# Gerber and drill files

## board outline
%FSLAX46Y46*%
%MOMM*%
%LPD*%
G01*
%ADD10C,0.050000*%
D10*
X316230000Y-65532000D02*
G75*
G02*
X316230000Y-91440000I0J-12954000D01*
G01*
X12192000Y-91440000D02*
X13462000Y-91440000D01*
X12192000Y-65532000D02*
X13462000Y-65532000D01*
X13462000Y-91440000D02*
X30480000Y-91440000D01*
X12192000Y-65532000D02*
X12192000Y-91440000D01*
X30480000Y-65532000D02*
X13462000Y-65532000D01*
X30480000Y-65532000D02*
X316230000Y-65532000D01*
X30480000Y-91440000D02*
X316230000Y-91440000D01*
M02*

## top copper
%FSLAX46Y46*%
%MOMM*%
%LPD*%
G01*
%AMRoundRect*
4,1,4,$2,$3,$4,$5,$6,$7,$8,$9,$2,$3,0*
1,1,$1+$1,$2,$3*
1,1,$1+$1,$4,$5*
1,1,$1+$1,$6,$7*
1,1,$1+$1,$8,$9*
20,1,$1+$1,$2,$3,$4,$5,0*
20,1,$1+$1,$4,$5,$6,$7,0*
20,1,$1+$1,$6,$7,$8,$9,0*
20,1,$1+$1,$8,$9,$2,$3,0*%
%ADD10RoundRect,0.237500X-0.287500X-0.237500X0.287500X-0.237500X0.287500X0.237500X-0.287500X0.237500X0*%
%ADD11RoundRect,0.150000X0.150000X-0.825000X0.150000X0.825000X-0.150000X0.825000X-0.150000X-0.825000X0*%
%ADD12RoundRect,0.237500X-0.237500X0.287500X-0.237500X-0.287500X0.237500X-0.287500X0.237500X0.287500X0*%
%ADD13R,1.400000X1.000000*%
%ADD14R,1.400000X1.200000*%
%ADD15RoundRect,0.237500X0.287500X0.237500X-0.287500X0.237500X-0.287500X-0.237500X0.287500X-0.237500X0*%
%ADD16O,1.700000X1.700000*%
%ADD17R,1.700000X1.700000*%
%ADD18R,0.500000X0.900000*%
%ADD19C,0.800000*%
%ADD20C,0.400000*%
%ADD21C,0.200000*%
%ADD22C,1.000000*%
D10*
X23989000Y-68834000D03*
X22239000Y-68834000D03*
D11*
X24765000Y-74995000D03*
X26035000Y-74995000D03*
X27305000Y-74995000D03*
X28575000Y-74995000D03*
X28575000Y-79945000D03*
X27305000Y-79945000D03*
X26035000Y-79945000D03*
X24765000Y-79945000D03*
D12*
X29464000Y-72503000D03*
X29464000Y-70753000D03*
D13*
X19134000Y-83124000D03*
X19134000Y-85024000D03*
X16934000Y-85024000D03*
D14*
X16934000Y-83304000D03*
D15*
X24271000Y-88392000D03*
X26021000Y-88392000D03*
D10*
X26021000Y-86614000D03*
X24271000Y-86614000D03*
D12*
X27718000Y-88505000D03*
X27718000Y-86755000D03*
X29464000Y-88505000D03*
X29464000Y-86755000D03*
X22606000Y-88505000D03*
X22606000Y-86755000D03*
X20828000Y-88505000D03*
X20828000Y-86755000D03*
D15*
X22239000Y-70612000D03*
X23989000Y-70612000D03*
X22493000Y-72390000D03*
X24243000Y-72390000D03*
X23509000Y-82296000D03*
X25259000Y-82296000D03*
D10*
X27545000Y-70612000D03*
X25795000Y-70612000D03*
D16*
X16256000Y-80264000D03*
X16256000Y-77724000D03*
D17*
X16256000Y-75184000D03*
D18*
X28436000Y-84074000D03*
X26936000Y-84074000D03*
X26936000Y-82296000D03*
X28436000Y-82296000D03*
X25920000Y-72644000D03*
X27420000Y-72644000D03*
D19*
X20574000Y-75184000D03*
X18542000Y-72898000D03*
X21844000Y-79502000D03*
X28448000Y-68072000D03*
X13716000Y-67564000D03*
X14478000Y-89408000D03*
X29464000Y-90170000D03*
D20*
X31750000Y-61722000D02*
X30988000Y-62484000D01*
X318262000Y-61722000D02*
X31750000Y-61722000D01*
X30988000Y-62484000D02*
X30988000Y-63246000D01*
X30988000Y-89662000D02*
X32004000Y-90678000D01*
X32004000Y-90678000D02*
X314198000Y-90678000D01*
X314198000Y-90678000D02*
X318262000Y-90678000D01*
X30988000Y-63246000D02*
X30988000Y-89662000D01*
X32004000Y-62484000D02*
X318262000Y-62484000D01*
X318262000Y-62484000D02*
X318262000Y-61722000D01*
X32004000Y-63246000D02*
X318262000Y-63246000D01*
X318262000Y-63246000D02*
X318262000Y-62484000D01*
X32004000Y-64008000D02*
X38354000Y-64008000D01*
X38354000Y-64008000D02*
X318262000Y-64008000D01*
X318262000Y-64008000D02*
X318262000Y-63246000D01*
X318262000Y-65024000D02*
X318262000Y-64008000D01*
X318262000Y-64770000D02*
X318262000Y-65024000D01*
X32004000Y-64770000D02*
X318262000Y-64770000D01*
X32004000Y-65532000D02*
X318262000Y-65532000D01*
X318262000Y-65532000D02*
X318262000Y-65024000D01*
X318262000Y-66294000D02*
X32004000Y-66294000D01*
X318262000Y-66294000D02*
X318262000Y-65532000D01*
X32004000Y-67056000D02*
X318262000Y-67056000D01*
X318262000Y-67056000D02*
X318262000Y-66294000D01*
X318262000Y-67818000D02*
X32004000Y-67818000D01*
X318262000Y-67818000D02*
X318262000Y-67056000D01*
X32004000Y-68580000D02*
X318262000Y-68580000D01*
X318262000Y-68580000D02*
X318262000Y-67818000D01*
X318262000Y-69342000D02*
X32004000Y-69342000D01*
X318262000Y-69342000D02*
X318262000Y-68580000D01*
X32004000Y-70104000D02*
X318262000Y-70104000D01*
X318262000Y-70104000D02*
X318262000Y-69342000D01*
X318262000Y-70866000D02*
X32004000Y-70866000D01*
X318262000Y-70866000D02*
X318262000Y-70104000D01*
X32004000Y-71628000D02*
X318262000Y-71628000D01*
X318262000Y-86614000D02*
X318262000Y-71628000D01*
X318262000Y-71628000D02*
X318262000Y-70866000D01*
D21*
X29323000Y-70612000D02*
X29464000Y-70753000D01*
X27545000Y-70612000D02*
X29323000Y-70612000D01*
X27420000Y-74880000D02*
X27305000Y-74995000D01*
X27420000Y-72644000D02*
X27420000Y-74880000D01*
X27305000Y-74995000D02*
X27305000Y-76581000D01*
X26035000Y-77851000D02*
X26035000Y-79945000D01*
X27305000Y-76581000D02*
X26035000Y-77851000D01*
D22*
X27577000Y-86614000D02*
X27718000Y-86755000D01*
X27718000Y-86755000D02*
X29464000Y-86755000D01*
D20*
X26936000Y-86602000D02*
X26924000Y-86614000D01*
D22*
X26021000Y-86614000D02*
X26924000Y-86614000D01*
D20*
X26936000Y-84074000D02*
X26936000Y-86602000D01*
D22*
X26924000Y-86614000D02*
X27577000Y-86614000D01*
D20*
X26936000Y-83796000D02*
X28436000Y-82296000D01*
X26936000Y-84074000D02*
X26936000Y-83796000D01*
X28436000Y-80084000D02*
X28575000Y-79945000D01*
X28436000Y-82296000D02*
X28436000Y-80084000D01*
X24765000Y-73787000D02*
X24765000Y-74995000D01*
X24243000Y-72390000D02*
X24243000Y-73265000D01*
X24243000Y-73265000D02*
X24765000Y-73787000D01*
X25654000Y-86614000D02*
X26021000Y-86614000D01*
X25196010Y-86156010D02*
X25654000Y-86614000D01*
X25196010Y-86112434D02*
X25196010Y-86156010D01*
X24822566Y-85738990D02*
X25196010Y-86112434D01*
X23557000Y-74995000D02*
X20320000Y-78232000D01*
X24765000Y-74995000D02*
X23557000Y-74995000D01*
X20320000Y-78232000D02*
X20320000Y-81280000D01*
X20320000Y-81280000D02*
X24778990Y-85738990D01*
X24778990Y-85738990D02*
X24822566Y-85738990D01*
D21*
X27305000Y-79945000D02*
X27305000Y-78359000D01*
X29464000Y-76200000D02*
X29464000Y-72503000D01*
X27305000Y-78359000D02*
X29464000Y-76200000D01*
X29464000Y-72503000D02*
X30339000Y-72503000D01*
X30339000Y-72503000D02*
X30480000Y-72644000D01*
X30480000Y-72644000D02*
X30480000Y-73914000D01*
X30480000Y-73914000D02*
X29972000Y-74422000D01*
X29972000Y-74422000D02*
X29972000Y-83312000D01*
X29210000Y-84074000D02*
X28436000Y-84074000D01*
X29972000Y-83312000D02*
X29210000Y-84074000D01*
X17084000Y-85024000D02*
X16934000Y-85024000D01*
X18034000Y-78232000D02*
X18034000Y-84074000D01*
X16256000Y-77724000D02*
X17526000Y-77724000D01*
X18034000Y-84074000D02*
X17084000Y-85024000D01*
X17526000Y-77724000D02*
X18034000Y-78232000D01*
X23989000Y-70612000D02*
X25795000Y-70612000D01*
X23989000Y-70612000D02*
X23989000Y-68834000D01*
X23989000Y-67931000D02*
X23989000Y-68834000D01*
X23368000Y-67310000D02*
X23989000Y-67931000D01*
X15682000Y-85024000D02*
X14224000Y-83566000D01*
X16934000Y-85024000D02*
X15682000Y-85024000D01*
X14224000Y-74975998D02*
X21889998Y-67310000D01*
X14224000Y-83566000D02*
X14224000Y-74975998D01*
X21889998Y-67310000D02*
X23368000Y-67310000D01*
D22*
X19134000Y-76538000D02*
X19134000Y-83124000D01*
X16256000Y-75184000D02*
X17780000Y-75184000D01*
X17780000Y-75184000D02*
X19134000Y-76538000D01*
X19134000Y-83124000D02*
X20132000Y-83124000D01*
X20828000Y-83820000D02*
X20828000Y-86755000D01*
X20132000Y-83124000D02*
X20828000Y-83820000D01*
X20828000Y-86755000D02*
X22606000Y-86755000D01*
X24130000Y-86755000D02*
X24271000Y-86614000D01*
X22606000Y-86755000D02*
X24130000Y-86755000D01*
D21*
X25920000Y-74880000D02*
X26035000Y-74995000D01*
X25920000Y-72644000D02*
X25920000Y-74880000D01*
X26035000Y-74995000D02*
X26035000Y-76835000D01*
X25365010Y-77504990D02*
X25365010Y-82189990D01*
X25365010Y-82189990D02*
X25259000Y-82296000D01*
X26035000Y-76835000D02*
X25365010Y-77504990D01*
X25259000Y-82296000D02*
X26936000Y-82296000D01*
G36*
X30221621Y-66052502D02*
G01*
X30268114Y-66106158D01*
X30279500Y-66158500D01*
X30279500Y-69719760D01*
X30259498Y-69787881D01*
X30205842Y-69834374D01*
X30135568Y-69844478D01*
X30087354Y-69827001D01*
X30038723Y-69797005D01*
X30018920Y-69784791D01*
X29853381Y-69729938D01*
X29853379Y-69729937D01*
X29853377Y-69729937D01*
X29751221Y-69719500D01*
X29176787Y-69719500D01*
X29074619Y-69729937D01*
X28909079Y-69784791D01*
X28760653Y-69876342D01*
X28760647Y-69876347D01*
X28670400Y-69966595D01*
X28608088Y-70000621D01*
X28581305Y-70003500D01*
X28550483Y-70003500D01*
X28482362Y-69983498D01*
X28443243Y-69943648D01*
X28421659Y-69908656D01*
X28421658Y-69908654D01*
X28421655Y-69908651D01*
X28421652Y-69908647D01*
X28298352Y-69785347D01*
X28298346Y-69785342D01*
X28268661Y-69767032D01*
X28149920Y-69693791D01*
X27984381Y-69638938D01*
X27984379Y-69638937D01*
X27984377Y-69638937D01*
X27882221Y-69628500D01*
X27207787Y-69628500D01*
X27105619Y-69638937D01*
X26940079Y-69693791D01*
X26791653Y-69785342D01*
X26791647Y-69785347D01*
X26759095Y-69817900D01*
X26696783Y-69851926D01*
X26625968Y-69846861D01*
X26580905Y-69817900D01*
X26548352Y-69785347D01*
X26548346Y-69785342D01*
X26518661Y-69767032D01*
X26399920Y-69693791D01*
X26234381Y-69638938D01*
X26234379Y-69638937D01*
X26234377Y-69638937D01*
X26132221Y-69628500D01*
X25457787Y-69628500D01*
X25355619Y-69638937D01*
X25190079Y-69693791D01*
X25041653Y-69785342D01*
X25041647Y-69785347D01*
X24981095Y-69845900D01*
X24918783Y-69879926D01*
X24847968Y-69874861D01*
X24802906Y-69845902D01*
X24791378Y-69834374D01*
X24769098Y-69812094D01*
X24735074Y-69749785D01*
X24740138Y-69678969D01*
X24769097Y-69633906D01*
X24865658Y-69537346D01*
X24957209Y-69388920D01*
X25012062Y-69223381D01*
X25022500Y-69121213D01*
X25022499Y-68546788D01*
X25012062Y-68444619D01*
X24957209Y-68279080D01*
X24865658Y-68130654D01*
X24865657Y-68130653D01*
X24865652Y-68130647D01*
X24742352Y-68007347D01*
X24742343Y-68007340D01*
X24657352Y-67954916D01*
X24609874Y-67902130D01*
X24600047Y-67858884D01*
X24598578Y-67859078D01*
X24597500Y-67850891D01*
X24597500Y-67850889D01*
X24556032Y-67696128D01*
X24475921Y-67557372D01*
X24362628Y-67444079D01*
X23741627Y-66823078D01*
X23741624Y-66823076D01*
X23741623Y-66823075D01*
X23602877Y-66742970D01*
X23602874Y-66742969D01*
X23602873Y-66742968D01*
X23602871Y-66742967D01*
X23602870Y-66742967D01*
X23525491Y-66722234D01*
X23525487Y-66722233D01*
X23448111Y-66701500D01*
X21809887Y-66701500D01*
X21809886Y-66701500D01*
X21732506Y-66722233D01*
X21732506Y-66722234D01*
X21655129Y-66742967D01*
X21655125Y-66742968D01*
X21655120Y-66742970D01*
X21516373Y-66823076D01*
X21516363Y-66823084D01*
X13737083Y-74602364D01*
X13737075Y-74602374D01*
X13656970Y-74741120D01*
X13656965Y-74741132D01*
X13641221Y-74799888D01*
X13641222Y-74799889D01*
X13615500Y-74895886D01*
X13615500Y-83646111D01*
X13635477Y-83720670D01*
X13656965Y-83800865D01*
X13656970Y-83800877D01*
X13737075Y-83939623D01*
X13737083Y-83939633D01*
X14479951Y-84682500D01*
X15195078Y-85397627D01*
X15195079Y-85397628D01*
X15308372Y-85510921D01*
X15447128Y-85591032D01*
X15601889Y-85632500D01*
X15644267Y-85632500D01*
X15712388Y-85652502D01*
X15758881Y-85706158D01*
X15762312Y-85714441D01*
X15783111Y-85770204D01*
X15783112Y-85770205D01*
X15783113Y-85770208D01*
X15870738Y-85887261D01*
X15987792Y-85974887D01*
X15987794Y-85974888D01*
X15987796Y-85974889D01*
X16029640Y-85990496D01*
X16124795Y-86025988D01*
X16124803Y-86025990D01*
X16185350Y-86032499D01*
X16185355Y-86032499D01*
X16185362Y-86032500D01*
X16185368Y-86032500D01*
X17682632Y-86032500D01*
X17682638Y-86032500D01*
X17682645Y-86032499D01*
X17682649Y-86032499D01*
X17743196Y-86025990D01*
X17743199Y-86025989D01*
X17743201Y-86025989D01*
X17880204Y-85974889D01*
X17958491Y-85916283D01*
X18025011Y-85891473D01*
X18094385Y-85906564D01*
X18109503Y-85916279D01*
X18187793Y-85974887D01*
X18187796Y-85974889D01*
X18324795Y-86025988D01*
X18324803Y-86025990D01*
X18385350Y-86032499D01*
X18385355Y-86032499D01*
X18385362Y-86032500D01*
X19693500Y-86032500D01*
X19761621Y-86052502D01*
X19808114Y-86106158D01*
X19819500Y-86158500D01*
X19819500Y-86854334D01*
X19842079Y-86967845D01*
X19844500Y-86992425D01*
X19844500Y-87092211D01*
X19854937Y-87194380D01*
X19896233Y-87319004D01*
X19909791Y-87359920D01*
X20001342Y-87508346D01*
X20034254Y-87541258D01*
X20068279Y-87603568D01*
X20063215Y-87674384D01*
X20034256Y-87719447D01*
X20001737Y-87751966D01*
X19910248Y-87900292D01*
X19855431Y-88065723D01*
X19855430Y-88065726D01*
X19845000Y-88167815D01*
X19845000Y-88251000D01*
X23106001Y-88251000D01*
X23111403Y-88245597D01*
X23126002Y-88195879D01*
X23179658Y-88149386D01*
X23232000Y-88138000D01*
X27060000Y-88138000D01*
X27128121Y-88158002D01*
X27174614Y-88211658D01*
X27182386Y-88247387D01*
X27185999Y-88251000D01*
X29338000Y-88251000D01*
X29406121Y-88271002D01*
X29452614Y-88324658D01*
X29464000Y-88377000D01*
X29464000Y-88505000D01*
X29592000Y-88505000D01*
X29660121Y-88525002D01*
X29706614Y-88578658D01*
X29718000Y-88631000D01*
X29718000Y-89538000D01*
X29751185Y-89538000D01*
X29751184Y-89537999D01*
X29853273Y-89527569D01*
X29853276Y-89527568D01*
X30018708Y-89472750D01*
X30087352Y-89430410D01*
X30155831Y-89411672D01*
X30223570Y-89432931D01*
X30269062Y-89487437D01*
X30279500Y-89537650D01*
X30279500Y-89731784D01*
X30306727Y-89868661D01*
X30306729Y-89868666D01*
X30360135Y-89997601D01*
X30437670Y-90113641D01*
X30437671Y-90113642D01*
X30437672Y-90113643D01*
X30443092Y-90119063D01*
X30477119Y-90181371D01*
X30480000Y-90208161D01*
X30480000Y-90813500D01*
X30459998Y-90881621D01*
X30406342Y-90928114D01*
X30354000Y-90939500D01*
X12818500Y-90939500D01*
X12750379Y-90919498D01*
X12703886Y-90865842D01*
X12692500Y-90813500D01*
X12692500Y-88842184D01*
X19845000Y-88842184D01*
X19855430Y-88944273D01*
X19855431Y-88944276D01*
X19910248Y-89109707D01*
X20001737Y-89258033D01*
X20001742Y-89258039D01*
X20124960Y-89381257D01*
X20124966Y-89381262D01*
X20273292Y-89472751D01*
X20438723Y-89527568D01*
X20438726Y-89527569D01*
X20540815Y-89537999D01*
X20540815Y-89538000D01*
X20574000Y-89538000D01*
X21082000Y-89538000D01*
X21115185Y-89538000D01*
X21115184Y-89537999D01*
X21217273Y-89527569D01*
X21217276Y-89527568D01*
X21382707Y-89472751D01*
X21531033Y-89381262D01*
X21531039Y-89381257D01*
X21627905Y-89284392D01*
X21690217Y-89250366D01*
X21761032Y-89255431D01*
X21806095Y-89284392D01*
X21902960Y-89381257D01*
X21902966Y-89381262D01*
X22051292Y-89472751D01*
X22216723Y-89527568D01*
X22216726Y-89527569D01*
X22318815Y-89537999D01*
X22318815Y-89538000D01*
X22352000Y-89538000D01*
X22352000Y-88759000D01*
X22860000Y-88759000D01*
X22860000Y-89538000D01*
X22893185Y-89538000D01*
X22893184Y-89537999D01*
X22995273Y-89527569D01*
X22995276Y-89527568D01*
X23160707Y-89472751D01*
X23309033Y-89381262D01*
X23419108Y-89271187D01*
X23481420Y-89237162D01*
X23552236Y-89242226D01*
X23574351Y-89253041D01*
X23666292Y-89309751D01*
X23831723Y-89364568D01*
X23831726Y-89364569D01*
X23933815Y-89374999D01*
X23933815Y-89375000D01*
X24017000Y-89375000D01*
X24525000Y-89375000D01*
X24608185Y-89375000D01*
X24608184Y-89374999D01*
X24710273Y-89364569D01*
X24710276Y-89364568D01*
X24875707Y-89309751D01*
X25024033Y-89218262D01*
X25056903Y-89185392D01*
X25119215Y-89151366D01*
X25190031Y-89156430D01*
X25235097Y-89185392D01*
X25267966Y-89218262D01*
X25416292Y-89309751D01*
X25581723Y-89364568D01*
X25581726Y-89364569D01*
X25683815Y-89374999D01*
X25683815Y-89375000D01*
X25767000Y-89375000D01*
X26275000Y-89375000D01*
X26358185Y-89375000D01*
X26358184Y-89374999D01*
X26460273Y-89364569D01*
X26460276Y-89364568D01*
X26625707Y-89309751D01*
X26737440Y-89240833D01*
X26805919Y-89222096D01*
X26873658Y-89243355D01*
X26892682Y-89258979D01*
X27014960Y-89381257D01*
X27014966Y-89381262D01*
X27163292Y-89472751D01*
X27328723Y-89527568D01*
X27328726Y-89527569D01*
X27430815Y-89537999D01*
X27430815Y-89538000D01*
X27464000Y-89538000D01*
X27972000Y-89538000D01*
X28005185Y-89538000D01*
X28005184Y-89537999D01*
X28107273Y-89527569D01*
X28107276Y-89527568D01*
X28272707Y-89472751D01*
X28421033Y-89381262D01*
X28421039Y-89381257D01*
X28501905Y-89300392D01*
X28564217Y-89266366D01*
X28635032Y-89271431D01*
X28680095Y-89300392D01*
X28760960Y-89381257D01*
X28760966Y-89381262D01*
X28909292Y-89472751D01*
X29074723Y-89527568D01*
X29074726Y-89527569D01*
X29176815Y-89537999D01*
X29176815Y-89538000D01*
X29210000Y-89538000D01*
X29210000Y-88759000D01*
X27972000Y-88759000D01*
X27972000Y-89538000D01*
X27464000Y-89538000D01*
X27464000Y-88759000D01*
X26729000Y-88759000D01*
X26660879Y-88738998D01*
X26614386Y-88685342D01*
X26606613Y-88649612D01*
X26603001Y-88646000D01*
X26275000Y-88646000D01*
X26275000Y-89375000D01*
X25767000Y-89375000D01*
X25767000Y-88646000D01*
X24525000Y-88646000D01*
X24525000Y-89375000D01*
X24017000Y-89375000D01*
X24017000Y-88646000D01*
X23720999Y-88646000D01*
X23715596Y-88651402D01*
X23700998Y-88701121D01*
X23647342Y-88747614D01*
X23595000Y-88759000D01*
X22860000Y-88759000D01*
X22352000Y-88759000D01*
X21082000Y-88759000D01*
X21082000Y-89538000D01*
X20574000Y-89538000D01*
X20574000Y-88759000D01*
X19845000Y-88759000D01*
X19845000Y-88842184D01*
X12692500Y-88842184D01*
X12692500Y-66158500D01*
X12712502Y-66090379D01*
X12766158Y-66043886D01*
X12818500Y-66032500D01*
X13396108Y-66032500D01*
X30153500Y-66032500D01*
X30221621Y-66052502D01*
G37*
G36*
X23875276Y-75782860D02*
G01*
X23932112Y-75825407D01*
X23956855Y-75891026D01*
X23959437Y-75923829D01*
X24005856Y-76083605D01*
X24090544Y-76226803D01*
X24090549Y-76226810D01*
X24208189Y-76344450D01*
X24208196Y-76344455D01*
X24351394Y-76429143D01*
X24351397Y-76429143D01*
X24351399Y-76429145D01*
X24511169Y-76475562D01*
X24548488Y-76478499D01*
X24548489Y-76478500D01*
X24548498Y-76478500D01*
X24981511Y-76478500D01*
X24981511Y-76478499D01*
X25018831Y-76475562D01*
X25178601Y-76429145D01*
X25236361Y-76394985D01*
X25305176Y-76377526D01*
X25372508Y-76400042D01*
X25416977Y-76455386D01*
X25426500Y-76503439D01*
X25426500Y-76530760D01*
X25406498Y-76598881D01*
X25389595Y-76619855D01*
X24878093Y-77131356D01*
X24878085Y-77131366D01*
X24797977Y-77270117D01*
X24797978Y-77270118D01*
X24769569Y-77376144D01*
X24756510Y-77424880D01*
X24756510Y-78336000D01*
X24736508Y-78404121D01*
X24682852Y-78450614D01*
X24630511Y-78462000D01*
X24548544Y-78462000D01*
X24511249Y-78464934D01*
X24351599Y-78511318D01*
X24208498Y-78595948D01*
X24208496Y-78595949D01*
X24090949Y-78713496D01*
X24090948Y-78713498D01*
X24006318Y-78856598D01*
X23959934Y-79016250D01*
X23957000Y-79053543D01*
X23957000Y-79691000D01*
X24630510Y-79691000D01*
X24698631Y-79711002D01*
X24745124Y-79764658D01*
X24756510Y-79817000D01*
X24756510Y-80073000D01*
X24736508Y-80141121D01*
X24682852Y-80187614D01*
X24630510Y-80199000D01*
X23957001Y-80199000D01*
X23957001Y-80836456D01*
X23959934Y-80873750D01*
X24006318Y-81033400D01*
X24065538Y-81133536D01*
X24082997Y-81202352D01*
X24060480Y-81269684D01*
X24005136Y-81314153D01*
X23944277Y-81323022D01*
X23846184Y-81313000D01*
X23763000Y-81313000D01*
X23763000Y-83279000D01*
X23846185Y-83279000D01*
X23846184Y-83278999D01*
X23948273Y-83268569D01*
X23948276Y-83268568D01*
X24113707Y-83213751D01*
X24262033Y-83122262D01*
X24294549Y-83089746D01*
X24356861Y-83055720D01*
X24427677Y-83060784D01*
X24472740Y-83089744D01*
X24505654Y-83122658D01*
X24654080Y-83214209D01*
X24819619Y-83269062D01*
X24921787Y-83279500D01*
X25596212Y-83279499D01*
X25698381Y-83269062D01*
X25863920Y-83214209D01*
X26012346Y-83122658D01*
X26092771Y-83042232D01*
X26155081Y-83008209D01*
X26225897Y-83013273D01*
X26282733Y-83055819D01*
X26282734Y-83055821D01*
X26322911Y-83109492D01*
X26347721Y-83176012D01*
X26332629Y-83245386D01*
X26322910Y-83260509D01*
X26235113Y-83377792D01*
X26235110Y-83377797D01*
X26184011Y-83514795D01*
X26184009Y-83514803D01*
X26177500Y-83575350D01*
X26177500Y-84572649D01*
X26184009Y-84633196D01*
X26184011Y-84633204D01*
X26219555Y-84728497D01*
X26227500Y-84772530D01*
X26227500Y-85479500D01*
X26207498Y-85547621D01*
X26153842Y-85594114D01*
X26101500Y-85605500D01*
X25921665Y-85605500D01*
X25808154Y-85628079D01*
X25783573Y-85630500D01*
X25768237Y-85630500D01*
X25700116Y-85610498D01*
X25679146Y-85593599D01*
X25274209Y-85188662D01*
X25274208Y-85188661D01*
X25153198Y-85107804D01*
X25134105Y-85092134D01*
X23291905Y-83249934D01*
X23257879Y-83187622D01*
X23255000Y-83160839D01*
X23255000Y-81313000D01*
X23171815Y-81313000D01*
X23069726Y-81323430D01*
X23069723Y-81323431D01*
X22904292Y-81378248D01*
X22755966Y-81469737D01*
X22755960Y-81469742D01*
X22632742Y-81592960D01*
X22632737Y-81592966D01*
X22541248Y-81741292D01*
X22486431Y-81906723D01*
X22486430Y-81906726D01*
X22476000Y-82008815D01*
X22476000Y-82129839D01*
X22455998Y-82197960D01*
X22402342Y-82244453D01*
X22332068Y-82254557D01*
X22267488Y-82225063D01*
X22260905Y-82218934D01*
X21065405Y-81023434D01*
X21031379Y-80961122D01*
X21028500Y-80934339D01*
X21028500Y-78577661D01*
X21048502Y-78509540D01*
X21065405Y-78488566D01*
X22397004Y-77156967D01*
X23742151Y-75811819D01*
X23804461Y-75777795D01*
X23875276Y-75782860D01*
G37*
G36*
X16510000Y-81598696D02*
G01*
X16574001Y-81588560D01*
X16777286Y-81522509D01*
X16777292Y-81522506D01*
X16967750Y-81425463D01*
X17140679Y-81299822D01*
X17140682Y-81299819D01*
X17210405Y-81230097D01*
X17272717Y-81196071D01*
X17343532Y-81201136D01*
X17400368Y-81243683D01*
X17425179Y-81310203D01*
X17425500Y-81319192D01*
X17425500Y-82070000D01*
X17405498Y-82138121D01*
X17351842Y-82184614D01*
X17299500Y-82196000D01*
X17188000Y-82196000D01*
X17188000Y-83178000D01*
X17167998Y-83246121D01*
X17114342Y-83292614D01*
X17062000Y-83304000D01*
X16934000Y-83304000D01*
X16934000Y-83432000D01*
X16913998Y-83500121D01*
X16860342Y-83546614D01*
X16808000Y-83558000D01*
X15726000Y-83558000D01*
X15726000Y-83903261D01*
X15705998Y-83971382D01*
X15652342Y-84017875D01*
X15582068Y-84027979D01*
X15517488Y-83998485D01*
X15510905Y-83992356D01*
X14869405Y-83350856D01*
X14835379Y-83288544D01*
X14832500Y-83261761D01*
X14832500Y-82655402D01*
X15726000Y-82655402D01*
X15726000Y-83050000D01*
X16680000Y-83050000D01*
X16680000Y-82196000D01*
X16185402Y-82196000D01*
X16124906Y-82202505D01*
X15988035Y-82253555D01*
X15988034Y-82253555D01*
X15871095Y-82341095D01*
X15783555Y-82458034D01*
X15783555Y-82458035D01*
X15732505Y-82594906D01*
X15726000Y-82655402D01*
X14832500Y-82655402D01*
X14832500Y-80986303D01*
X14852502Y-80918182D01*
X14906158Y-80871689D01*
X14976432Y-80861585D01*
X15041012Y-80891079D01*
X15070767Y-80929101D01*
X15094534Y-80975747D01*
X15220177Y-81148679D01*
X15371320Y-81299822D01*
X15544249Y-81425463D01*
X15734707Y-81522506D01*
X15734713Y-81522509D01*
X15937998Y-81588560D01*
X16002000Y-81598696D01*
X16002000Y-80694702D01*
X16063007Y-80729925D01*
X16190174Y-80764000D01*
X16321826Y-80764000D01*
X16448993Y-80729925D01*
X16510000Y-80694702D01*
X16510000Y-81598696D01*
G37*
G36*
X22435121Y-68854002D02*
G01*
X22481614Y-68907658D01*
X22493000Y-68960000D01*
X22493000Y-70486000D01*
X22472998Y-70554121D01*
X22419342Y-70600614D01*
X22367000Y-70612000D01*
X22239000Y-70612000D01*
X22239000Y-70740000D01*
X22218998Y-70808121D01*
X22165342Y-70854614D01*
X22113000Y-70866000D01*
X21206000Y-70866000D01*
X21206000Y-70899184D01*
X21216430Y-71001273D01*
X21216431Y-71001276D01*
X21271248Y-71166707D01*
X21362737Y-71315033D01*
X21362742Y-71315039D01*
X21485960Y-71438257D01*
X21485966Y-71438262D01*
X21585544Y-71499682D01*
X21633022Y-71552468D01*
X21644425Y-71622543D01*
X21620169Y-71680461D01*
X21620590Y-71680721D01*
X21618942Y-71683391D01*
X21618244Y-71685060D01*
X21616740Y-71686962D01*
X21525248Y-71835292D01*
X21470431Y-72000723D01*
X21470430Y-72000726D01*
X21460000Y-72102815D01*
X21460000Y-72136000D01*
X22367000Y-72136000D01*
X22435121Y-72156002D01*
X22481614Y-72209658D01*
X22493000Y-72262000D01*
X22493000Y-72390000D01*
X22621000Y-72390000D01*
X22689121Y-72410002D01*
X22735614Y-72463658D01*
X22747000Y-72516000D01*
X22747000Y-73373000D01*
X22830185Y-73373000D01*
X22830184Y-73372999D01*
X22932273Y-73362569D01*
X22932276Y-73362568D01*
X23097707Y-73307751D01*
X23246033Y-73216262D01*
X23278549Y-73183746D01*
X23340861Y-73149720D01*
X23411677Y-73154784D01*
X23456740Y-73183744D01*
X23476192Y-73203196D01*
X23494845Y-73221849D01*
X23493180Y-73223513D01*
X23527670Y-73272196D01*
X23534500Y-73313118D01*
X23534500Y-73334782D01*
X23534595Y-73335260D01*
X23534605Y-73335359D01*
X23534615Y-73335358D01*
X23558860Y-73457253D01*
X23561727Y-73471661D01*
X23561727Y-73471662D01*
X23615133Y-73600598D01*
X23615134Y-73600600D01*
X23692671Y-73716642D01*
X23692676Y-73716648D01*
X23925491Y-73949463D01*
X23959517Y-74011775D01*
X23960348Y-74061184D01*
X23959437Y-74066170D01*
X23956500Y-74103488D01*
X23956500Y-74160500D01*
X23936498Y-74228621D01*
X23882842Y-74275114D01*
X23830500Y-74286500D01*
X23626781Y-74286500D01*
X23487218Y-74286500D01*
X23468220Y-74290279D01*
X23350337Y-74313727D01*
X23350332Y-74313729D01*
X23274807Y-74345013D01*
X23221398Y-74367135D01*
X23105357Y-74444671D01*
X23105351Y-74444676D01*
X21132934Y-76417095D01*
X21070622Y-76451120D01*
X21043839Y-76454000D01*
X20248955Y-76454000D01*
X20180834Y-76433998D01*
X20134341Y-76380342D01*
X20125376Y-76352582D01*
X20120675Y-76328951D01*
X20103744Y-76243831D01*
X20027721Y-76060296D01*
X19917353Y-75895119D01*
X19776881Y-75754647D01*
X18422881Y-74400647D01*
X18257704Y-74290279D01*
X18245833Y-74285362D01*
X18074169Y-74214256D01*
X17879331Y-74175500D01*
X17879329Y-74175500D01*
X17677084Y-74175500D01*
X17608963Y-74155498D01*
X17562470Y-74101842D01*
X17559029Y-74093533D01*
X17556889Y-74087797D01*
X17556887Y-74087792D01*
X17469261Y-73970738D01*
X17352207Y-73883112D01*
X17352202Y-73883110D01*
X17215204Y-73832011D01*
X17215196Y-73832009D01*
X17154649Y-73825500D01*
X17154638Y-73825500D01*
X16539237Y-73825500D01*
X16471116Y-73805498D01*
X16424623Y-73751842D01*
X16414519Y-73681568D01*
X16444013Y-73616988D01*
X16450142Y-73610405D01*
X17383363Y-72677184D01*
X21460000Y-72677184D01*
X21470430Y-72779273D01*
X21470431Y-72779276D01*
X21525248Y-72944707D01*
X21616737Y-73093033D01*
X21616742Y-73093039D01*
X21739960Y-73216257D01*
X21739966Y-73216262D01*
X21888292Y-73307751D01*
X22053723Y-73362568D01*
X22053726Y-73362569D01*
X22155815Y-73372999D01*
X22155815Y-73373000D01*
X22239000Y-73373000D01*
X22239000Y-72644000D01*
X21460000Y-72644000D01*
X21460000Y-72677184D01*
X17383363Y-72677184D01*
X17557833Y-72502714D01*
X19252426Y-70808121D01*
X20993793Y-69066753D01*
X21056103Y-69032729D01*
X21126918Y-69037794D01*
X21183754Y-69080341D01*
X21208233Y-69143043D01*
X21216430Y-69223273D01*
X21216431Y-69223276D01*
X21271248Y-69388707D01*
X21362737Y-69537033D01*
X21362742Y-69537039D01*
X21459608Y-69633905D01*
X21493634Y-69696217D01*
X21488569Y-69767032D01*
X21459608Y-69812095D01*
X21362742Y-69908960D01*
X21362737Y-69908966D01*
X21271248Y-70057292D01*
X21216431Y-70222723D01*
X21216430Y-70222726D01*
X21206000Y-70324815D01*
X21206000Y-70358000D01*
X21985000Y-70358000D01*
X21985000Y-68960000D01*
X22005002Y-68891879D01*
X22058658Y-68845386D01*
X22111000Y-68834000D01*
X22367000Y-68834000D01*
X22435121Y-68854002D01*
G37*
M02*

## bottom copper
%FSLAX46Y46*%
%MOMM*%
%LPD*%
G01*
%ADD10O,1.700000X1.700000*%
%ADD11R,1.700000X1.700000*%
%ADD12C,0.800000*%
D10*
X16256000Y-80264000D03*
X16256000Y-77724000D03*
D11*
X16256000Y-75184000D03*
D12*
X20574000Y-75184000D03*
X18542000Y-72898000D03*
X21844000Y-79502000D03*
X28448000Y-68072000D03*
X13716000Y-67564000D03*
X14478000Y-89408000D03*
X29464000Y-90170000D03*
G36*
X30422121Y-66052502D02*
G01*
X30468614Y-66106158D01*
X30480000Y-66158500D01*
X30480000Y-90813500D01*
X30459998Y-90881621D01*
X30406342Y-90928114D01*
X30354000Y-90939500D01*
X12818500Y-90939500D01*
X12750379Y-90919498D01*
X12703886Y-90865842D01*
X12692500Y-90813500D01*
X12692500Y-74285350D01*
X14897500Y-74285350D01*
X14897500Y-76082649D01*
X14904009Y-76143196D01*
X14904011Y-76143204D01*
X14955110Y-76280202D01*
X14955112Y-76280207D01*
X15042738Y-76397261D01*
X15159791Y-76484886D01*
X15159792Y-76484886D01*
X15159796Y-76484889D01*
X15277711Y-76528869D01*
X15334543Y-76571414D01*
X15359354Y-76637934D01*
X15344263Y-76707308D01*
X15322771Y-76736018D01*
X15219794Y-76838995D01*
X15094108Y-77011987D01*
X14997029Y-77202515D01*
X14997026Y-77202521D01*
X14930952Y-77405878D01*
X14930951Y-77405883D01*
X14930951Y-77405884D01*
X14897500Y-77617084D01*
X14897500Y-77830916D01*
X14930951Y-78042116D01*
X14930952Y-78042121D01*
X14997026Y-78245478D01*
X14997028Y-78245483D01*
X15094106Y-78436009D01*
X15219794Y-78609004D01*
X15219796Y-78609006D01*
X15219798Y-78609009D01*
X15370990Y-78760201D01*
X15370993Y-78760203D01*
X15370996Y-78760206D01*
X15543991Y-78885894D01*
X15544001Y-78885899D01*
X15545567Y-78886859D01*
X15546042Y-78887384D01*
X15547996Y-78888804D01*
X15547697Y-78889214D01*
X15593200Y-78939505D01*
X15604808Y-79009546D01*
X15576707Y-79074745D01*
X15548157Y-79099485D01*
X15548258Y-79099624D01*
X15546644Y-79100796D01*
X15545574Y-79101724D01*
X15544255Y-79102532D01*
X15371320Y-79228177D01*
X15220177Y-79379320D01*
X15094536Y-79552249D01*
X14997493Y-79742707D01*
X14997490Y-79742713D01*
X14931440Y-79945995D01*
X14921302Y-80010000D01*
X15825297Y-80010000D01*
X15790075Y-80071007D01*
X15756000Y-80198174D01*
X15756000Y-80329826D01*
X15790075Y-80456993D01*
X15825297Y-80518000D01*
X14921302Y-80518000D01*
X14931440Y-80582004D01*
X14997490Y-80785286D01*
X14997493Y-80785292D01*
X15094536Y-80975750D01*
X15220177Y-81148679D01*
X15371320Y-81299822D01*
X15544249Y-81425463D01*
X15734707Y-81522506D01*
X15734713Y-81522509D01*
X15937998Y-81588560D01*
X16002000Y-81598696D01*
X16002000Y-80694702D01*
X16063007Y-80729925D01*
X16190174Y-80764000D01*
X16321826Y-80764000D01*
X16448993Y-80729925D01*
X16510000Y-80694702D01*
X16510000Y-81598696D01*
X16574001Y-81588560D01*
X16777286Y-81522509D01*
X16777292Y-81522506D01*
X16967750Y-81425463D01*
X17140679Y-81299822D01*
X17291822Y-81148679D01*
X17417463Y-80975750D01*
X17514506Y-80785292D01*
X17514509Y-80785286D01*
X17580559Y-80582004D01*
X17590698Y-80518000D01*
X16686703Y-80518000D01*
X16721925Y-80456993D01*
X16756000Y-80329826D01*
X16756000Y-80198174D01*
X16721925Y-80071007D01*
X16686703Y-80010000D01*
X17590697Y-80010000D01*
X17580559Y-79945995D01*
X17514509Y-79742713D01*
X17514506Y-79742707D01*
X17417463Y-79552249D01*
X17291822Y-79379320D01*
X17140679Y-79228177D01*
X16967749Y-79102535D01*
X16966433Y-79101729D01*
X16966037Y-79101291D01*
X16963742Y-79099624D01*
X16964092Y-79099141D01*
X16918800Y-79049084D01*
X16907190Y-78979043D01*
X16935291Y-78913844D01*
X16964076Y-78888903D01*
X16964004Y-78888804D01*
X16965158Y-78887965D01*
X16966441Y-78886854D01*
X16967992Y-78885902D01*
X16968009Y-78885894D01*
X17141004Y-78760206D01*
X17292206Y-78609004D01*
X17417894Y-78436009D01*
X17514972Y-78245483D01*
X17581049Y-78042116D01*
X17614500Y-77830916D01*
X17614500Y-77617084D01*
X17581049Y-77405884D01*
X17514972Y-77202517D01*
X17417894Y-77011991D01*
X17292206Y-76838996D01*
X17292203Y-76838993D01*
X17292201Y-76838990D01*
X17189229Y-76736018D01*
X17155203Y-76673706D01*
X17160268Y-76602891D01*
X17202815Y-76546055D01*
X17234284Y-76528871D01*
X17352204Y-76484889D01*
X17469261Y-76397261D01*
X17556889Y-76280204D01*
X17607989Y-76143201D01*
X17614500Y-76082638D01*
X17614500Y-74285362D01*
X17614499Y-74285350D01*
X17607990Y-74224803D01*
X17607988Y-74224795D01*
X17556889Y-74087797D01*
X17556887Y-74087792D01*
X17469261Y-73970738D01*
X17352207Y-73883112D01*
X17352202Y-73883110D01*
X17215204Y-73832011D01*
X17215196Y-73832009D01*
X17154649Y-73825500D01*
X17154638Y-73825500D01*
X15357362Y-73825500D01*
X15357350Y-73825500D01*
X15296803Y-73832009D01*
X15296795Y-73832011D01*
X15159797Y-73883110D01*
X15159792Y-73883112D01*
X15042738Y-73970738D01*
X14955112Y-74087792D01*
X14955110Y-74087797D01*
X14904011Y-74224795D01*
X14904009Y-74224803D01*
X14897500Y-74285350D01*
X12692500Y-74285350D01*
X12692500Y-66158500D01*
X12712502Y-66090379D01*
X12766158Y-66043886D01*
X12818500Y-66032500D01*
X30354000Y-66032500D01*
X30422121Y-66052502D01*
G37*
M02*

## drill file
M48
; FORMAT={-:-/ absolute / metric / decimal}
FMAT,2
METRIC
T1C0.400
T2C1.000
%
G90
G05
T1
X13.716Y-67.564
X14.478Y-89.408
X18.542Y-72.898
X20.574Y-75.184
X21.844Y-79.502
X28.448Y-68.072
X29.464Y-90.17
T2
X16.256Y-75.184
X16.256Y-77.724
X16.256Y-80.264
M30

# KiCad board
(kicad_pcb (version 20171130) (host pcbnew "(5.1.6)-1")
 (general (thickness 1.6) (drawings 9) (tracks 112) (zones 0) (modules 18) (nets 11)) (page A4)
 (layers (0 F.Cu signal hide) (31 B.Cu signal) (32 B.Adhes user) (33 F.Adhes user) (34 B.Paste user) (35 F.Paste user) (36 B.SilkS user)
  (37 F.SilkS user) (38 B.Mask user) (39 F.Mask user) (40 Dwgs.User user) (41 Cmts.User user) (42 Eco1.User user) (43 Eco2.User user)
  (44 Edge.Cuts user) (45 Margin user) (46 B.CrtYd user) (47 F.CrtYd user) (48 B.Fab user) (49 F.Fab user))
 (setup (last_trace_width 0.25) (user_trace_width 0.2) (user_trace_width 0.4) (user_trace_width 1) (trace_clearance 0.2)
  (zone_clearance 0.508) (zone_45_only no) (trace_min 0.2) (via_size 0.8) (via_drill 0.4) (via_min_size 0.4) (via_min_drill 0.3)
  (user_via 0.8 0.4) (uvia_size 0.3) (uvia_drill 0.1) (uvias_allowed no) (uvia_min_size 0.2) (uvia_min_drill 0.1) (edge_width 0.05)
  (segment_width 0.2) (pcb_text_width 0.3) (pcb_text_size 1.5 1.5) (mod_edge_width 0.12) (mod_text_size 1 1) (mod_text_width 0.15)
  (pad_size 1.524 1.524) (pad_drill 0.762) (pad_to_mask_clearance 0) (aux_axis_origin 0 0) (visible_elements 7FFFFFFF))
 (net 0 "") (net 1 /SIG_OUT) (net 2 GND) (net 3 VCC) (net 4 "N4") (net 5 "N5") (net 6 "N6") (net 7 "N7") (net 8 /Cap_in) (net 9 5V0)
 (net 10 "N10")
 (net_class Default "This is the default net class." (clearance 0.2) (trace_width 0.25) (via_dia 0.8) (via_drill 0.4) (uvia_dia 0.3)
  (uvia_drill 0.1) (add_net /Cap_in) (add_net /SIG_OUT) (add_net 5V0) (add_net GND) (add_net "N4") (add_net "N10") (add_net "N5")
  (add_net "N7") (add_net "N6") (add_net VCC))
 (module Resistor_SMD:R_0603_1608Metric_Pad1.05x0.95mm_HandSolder (layer F.Cu) (at 23.114 68.834)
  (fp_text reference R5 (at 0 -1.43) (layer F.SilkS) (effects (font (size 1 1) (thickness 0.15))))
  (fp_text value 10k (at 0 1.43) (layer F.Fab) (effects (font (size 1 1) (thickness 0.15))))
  (pad 2 smd roundrect (at 0.875 0) (size 1.05 0.95) (layers F.Cu F.Paste F.Mask) (roundrect_rratio 0.25) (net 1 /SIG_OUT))
  (pad 1 smd roundrect (at -0.875 0) (size 1.05 0.95) (layers F.Cu F.Paste F.Mask) (roundrect_rratio 0.25) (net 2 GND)))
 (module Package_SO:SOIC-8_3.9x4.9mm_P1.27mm (layer F.Cu) (at 26.67 77.47 90)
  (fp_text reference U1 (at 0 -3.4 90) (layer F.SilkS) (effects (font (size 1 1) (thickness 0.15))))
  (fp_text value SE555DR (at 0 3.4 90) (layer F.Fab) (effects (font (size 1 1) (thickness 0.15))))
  (pad 8 smd roundrect (at 2.475 -1.905 90) (size 1.95 0.6) (layers F.Cu F.Paste F.Mask) (roundrect_rratio 0.25) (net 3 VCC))
  (pad 7 smd roundrect (at 2.475 -0.635 90) (size 1.95 0.6) (layers F.Cu F.Paste F.Mask) (roundrect_rratio 0.25) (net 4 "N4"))
  (pad 6 smd roundrect (at 2.475 0.635 90) (size 1.95 0.6) (layers F.Cu F.Paste F.Mask) (roundrect_rratio 0.25) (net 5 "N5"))
  (pad 5 smd roundrect (at 2.475 1.905 90) (size 1.95 0.6) (layers F.Cu F.Paste F.Mask) (roundrect_rratio 0.25) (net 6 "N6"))
  (pad 4 smd roundrect (at -2.475 1.905 90) (size 1.95 0.6) (layers F.Cu F.Paste F.Mask) (roundrect_rratio 0.25) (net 3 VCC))
  (pad 3 smd roundrect (at -2.475 0.635 90) (size 1.95 0.6) (layers F.Cu F.Paste F.Mask) (roundrect_rratio 0.25) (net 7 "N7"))
  (pad 2 smd roundrect (at -2.475 -0.635 90) (size 1.95 0.6) (layers F.Cu F.Paste F.Mask) (roundrect_rratio 0.25) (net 5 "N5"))
  (pad 1 smd roundrect (at -2.475 -1.905 90) (size 1.95 0.6) (layers F.Cu F.Paste F.Mask) (roundrect_rratio 0.25) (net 2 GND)))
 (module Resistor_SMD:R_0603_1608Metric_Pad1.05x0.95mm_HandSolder (layer F.Cu) (at 29.464 71.628 270)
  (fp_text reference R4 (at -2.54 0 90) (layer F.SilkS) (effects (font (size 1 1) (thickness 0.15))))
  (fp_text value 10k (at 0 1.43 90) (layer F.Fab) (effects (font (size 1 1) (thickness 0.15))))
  (pad 2 smd roundrect (at 0.875 0 270) (size 1.05 0.95) (layers F.Cu F.Paste F.Mask) (roundrect_rratio 0.25) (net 7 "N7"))
  (pad 1 smd roundrect (at -0.875 0 270) (size 1.05 0.95) (layers F.Cu F.Paste F.Mask) (roundrect_rratio 0.25) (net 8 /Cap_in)))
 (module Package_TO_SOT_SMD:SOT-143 (layer F.Cu) (at 18.034 84.074)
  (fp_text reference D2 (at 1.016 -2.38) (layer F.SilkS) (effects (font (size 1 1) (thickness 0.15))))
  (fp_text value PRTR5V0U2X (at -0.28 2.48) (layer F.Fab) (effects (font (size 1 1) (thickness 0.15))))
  (pad 4 smd rect (at 1.1 -0.95 270) (size 1 1.4) (layers F.Cu F.Paste F.Mask) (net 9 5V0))
  (pad 3 smd rect (at 1.1 0.95 270) (size 1 1.4) (layers F.Cu F.Paste F.Mask) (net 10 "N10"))
  (pad 2 smd rect (at -1.1 0.95 270) (size 1 1.4) (layers F.Cu F.Paste F.Mask) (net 1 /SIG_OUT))
  (pad 1 smd rect (at -1.1 -0.77 270) (size 1.2 1.4) (layers F.Cu F.Paste F.Mask) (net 2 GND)))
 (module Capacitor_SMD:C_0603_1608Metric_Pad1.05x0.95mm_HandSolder (layer F.Cu) (at 25.146 88.392 180)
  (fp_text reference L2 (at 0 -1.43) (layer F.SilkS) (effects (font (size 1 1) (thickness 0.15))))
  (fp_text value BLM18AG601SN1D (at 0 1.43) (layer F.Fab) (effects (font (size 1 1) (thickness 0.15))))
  (pad 2 smd roundrect (at 0.875 0 180) (size 1.05 0.95) (layers F.Cu F.Paste F.Mask) (roundrect_rratio 0.25) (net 2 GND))
  (pad 1 smd roundrect (at -0.875 0 180) (size 1.05 0.95) (layers F.Cu F.Paste F.Mask) (roundrect_rratio 0.25) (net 2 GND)))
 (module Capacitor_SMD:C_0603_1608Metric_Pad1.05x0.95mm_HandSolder (layer F.Cu) (at 25.146 86.614)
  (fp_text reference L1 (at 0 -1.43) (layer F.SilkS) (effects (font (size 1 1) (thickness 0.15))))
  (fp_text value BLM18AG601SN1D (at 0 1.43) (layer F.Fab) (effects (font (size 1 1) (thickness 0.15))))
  (pad 2 smd roundrect (at 0.875 0) (size 1.05 0.95) (layers F.Cu F.Paste F.Mask) (roundrect_rratio 0.25) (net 3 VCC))
  (pad 1 smd roundrect (at -0.875 0) (size 1.05 0.95) (layers F.Cu F.Paste F.Mask) (roundrect_rratio 0.25) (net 9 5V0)))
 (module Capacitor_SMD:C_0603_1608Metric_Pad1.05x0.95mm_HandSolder (layer F.Cu) (at 27.718 87.63 270)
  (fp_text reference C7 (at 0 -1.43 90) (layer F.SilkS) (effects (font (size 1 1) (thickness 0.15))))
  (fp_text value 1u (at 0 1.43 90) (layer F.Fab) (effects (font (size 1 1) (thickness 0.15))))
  (pad 2 smd roundrect (at 0.875 0 270) (size 1.05 0.95) (layers F.Cu F.Paste F.Mask) (roundrect_rratio 0.25) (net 2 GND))
  (pad 1 smd roundrect (at -0.875 0 270) (size 1.05 0.95) (layers F.Cu F.Paste F.Mask) (roundrect_rratio 0.25) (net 3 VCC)))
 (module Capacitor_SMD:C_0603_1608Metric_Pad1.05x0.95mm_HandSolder (layer F.Cu) (at 29.464 87.63 270)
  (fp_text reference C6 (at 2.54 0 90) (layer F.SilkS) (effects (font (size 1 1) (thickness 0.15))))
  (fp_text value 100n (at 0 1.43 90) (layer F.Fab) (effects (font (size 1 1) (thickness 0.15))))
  (pad 2 smd roundrect (at 0.875 0 270) (size 1.05 0.95) (layers F.Cu F.Paste F.Mask) (roundrect_rratio 0.25) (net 2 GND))
  (pad 1 smd roundrect (at -0.875 0 270) (size 1.05 0.95) (layers F.Cu F.Paste F.Mask) (roundrect_rratio 0.25) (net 3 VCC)))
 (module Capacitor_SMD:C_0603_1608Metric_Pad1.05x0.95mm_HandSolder (layer F.Cu) (at 22.606 87.63 270)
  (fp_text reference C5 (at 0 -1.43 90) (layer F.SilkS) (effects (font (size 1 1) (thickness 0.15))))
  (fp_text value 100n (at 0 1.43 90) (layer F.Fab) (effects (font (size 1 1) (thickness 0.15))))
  (pad 2 smd roundrect (at 0.875 0 270) (size 1.05 0.95) (layers F.Cu F.Paste F.Mask) (roundrect_rratio 0.25) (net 2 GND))
  (pad 1 smd roundrect (at -0.875 0 270) (size 1.05 0.95) (layers F.Cu F.Paste F.Mask) (roundrect_rratio 0.25) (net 9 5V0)))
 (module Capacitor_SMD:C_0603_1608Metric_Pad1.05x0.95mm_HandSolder (layer F.Cu) (at 20.828 87.63 270)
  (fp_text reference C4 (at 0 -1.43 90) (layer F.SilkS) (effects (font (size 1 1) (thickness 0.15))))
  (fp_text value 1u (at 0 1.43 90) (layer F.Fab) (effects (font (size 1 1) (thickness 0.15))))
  (pad 2 smd roundrect (at 0.875 0 270) (size 1.05 0.95) (layers F.Cu F.Paste F.Mask) (roundrect_rratio 0.25) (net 2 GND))
  (pad 1 smd roundrect (at -0.875 0 270) (size 1.05 0.95) (layers F.Cu F.Paste F.Mask) (roundrect_rratio 0.25) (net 9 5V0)))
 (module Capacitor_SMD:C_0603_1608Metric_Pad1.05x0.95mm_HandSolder (layer F.Cu) (at 23.114 70.612 180)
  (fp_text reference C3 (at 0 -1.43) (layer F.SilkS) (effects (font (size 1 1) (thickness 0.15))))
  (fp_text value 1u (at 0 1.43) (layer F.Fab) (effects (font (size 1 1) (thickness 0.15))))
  (pad 2 smd roundrect (at 0.875 0 180) (size 1.05 0.95) (layers F.Cu F.Paste F.Mask) (roundrect_rratio 0.25) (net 2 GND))
  (pad 1 smd roundrect (at -0.875 0 180) (size 1.05 0.95) (layers F.Cu F.Paste F.Mask) (roundrect_rratio 0.25) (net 1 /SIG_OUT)))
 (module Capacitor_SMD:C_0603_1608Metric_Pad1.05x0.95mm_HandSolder (layer F.Cu) (at 23.368 72.39 180)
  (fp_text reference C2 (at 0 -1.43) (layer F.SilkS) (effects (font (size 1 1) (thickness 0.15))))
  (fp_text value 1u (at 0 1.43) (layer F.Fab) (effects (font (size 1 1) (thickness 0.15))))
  (pad 2 smd roundrect (at 0.875 0 180) (size 1.05 0.95) (layers F.Cu F.Paste F.Mask) (roundrect_rratio 0.25) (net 2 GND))
  (pad 1 smd roundrect (at -0.875 0 180) (size 1.05 0.95) (layers F.Cu F.Paste F.Mask) (roundrect_rratio 0.25) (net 3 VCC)))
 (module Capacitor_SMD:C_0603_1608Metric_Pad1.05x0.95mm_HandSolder (layer F.Cu) (at 24.384 82.296 180)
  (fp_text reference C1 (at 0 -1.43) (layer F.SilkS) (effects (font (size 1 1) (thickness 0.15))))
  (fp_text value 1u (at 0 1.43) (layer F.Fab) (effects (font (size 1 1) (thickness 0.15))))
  (pad 2 smd roundrect (at 0.875 0 180) (size 1.05 0.95) (layers F.Cu F.Paste F.Mask) (roundrect_rratio 0.25) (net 2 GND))
  (pad 1 smd roundrect (at -0.875 0 180) (size 1.05 0.95) (layers F.Cu F.Paste F.Mask) (roundrect_rratio 0.25) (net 4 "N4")))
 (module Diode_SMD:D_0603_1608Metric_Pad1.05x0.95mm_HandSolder (layer F.Cu) (at 26.67 70.612)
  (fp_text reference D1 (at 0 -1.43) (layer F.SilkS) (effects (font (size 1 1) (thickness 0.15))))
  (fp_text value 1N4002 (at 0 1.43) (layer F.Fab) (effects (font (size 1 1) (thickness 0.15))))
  (pad 2 smd roundrect (at 0.875 0) (size 1.05 0.95) (layers F.Cu F.Paste F.Mask) (roundrect_rratio 0.25) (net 8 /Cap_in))
  (pad 1 smd roundrect (at -0.875 0) (size 1.05 0.95) (layers F.Cu F.Paste F.Mask) (roundrect_rratio 0.25) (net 1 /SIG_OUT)))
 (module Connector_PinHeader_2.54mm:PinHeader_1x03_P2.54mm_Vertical (layer F.Cu) (at 16.256 75.184)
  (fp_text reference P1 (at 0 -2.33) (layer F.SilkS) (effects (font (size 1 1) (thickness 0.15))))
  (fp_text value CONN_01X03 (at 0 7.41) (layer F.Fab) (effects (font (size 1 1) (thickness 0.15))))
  (pad 3 thru_hole oval (at 0 5.08) (size 1.7 1.7) (drill 1) (layers *.Cu *.Mask) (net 2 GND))
  (pad 2 thru_hole oval (at 0 2.54) (size 1.7 1.7) (drill 1) (layers *.Cu *.Mask) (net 1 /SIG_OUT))
  (pad 1 thru_hole rect (at 0 0) (size 1.7 1.7) (drill 1) (layers *.Cu *.Mask) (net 9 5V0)))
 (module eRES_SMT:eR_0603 (layer F.Cu) (at 27.686 84.074)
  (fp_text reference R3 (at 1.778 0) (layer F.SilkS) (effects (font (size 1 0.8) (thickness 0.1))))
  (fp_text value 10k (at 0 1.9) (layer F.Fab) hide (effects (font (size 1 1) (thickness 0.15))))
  (pad 2 smd rect (at 0.75 0) (size 0.5 0.9) (layers F.Cu F.Paste F.Mask) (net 7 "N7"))
  (pad 1 smd rect (at -0.75 0) (size 0.5 0.9) (layers F.Cu F.Paste F.Mask) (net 3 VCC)))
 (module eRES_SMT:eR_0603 (layer F.Cu) (at 27.686 82.296 180)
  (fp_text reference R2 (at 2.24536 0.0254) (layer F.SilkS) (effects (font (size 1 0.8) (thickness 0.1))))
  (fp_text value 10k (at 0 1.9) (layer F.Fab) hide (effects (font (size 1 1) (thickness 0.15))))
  (pad 2 smd rect (at 0.75 0 180) (size 0.5 0.9) (layers F.Cu F.Paste F.Mask) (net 4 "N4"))
  (pad 1 smd rect (at -0.75 0 180) (size 0.5 0.9) (layers F.Cu F.Paste F.Mask) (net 3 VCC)))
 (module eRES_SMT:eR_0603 (layer F.Cu) (at 26.67 72.644 180)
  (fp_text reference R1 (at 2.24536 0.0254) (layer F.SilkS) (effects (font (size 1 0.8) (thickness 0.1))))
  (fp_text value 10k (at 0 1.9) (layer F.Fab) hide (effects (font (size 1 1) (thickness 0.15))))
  (pad 2 smd rect (at 0.75 0 180) (size 0.5 0.9) (layers F.Cu F.Paste F.Mask) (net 4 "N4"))
  (pad 1 smd rect (at -0.75 0 180) (size 0.5 0.9) (layers F.Cu F.Paste F.Mask) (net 5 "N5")))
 (gr_arc (start 316.23 78.486) (end 316.23 91.44) (angle -180) (layer Edge.Cuts) (width 0.05))
 (gr_line (start 12.192 91.44) (end 13.462 91.44) (layer Edge.Cuts) (width 0.05))
 (gr_line (start 12.192 65.532) (end 13.462 65.532) (layer Edge.Cuts) (width 0.05))
 (gr_line (start 13.462 91.44) (end 30.48 91.44) (layer Edge.Cuts) (width 0.05))
 (gr_line (start 12.192 65.532) (end 12.192 91.44) (layer Edge.Cuts) (width 0.05))
 (gr_line (start 30.48 65.532) (end 13.462 65.532) (layer Edge.Cuts) (width 0.05))
 (gr_line (start 30.48 65.532) (end 316.23 65.532) (layer Edge.Cuts) (width 0.05))
 (gr_line (start 30.48 91.44) (end 316.23 91.44) (layer Edge.Cuts) (width 0.05))
 (segment (start 31.75 61.722) (end 30.988 62.484) (width 0.4) (layer F.Cu) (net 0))
 (segment (start 318.262 61.722) (end 31.75 61.722) (width 0.4) (layer F.Cu) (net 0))
 (segment (start 30.988 62.484) (end 30.988 63.246) (width 0.4) (layer F.Cu) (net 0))
 (segment (start 30.988 89.662) (end 32.004 90.678) (width 0.4) (layer F.Cu) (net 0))
 (segment (start 32.004 90.678) (end 314.198 90.678) (width 0.4) (layer F.Cu) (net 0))
 (segment (start 314.198 90.678) (end 318.262 90.678) (width 0.4) (layer F.Cu) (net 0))
 (segment (start 30.988 63.246) (end 30.988 89.662) (width 0.4) (layer F.Cu) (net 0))
 (segment (start 32.004 62.484) (end 318.262 62.484) (width 0.4) (layer F.Cu) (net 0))
 (segment (start 318.262 62.484) (end 318.262 61.722) (width 0.4) (layer F.Cu) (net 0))
 (segment (start 32.004 63.246) (end 318.262 63.246) (width 0.4) (layer F.Cu) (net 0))
 (segment (start 318.262 63.246) (end 318.262 62.484) (width 0.4) (layer F.Cu) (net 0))
 (segment (start 32.004 64.008) (end 38.354 64.008) (width 0.4) (layer F.Cu) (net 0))
 (segment (start 38.354 64.008) (end 318.262 64.008) (width 0.4) (layer F.Cu) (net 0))
 (segment (start 318.262 64.008) (end 318.262 63.246) (width 0.4) (layer F.Cu) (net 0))
 (segment (start 318.262 65.024) (end 318.262 64.008) (width 0.4) (layer F.Cu) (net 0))
 (segment (start 318.262 64.77) (end 318.262 65.024) (width 0.4) (layer F.Cu) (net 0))
 (segment (start 32.004 64.77) (end 318.262 64.77) (width 0.4) (layer F.Cu) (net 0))
 (segment (start 32.004 65.532) (end 318.262 65.532) (width 0.4) (layer F.Cu) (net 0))
 (segment (start 318.262 65.532) (end 318.262 65.024) (width 0.4) (layer F.Cu) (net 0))
 (segment (start 318.262 66.294) (end 32.004 66.294) (width 0.4) (layer F.Cu) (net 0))
 (segment (start 318.262 66.294) (end 318.262 65.532) (width 0.4) (layer F.Cu) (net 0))
 (segment (start 32.004 67.056) (end 318.262 67.056) (width 0.4) (layer F.Cu) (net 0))
 (segment (start 318.262 67.056) (end 318.262 66.294) (width 0.4) (layer F.Cu) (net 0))
 (segment (start 318.262 67.818) (end 32.004 67.818) (width 0.4) (layer F.Cu) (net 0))
 (segment (start 318.262 67.818) (end 318.262 67.056) (width 0.4) (layer F.Cu) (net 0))
 (segment (start 32.004 68.58) (end 318.262 68.58) (width 0.4) (layer F.Cu) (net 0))
 (segment (start 318.262 68.58) (end 318.262 67.818) (width 0.4) (layer F.Cu) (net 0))
 (segment (start 318.262 69.342) (end 32.004 69.342) (width 0.4) (layer F.Cu) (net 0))
 (segment (start 318.262 69.342) (end 318.262 68.58) (width 0.4) (layer F.Cu) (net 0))
 (segment (start 32.004 70.104) (end 318.262 70.104) (width 0.4) (layer F.Cu) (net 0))
 (segment (start 318.262 70.104) (end 318.262 69.342) (width 0.4) (layer F.Cu) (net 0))
 (segment (start 318.262 70.866) (end 32.004 70.866) (width 0.4) (layer F.Cu) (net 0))
 (segment (start 318.262 70.866) (end 318.262 70.104) (width 0.4) (layer F.Cu) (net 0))
 (segment (start 32.004 71.628) (end 318.262 71.628) (width 0.4) (layer F.Cu) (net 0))
 (segment (start 318.262 86.614) (end 318.262 71.628) (width 0.4) (layer F.Cu) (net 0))
 (segment (start 318.262 71.628) (end 318.262 70.866) (width 0.4) (layer F.Cu) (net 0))
 (segment (start 29.323 70.612) (end 29.464 70.753) (width 0.2) (layer F.Cu) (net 8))
 (segment (start 27.545 70.612) (end 29.323 70.612) (width 0.2) (layer F.Cu) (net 8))
 (segment (start 27.42 74.88) (end 27.305 74.995) (width 0.2) (layer F.Cu) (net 5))
 (segment (start 27.42 72.644) (end 27.42 74.88) (width 0.2) (layer F.Cu) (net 5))
 (segment (start 27.305 74.995) (end 27.305 76.581) (width 0.2) (layer F.Cu) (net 5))
 (segment (start 26.035 77.851) (end 26.035 79.945) (width 0.2) (layer F.Cu) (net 5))
 (segment (start 27.305 76.581) (end 26.035 77.851) (width 0.2) (layer F.Cu) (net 5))
 (segment (start 27.577 86.614) (end 27.718 86.755) (width 1) (layer F.Cu) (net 3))
 (segment (start 27.718 86.755) (end 29.464 86.755) (width 1) (layer F.Cu) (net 3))
 (segment (start 26.936 86.602) (end 26.924 86.614) (width 0.4) (layer F.Cu) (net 3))
 (segment (start 26.021 86.614) (end 26.924 86.614) (width 1) (layer F.Cu) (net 3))
 (segment (start 26.936 84.074) (end 26.936 86.602) (width 0.4) (layer F.Cu) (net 3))
 (segment (start 26.924 86.614) (end 27.577 86.614) (width 1) (layer F.Cu) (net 3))
 (segment (start 26.936 83.796) (end 28.436 82.296) (width 0.4) (layer F.Cu) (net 3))
 (segment (start 26.936 84.074) (end 26.936 83.796) (width 0.4) (layer F.Cu) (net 3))
 (segment (start 28.436 80.084) (end 28.575 79.945) (width 0.4) (layer F.Cu) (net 3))
 (segment (start 28.436 82.296) (end 28.436 80.084) (width 0.4) (layer F.Cu) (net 3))
 (segment (start 24.765 73.787) (end 24.765 74.995) (width 0.4) (layer F.Cu) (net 3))
 (segment (start 24.243 72.39) (end 24.243 73.265) (width 0.4) (layer F.Cu) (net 3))
 (segment (start 24.243 73.265) (end 24.765 73.787) (width 0.4) (layer F.Cu) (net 3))
 (segment (start 25.654 86.614) (end 26.021 86.614) (width 0.4) (layer F.Cu) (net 3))
 (segment (start 25.19601 86.15601) (end 25.654 86.614) (width 0.4) (layer F.Cu) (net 3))
 (segment (start 25.19601 86.112434) (end 25.19601 86.15601) (width 0.4) (layer F.Cu) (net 3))
 (segment (start 24.822566 85.73899) (end 25.19601 86.112434) (width 0.4) (layer F.Cu) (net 3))
 (segment (start 23.557 74.995) (end 20.32 78.232) (width 0.4) (layer F.Cu) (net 3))
 (segment (start 24.765 74.995) (end 23.557 74.995) (width 0.4) (layer F.Cu) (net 3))
 (segment (start 20.32 78.232) (end 20.32 81.28) (width 0.4) (layer F.Cu) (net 3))
 (segment (start 20.32 81.28) (end 24.77899 85.73899) (width 0.4) (layer F.Cu) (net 3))
 (segment (start 24.77899 85.73899) (end 24.822566 85.73899) (width 0.4) (layer F.Cu) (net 3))
 (segment (start 27.305 79.945) (end 27.305 78.359) (width 0.2) (layer F.Cu) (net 7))
 (segment (start 29.464 76.2) (end 29.464 72.503) (width 0.2) (layer F.Cu) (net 7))
 (segment (start 27.305 78.359) (end 29.464 76.2) (width 0.2) (layer F.Cu) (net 7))
 (segment (start 29.464 72.503) (end 30.339 72.503) (width 0.2) (layer F.Cu) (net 7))
 (segment (start 30.339 72.503) (end 30.48 72.644) (width 0.2) (layer F.Cu) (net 7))
 (segment (start 30.48 72.644) (end 30.48 73.914) (width 0.2) (layer F.Cu) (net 7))
 (segment (start 30.48 73.914) (end 29.972 74.422) (width 0.2) (layer F.Cu) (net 7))
 (segment (start 29.972 74.422) (end 29.972 83.312) (width 0.2) (layer F.Cu) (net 7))
 (segment (start 29.21 84.074) (end 28.436 84.074) (width 0.2) (layer F.Cu) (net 7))
 (segment (start 29.972 83.312) (end 29.21 84.074) (width 0.2) (layer F.Cu) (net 7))
 (via (at 20.574 75.184) (size 0.8) (drill 0.4) (layers F.Cu B.Cu) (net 2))
 (via (at 18.542 72.898) (size 0.8) (drill 0.4) (layers F.Cu B.Cu) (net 2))
 (via (at 21.844 79.502) (size 0.8) (drill 0.4) (layers F.Cu B.Cu) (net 2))
 (via (at 28.448 68.072) (size 0.8) (drill 0.4) (layers F.Cu B.Cu) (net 2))
 (via (at 13.716 67.564) (size 0.8) (drill 0.4) (layers F.Cu B.Cu) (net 2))
 (via (at 14.478 89.408) (size 0.8) (drill 0.4) (layers F.Cu B.Cu) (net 2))
 (via (at 29.464 90.17) (size 0.8) (drill 0.4) (layers F.Cu B.Cu) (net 2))
 (segment (start 17.084 85.024) (end 16.934 85.024) (width 0.2) (layer F.Cu) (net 1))
 (segment (start 18.034 78.232) (end 18.034 84.074) (width 0.2) (layer F.Cu) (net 1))
 (segment (start 16.256 77.724) (end 17.526 77.724) (width 0.2) (layer F.Cu) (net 1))
 (segment (start 18.034 84.074) (end 17.084 85.024) (width 0.2) (layer F.Cu) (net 1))
 (segment (start 17.526 77.724) (end 18.034 78.232) (width 0.2) (layer F.Cu) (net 1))
 (segment (start 23.989 70.612) (end 25.795 70.612) (width 0.2) (layer F.Cu) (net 1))
 (segment (start 23.989 70.612) (end 23.989 68.834) (width 0.2) (layer F.Cu) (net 1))
 (segment (start 23.989 67.931) (end 23.989 68.834) (width 0.2) (layer F.Cu) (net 1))
 (segment (start 23.368 67.31) (end 23.989 67.931) (width 0.2) (layer F.Cu) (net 1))
 (segment (start 15.682 85.024) (end 14.224 83.566) (width 0.2) (layer F.Cu) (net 1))
 (segment (start 16.934 85.024) (end 15.682 85.024) (width 0.2) (layer F.Cu) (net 1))
 (segment (start 14.224 74.975998) (end 21.889998 67.31) (width 0.2) (layer F.Cu) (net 1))
 (segment (start 14.224 83.566) (end 14.224 74.975998) (width 0.2) (layer F.Cu) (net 1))
 (segment (start 21.889998 67.31) (end 23.368 67.31) (width 0.2) (layer F.Cu) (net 1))
 (segment (start 19.134 76.538) (end 19.134 83.124) (width 1) (layer F.Cu) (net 9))
 (segment (start 16.256 75.184) (end 17.78 75.184) (width 1) (layer F.Cu) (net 9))
 (segment (start 17.78 75.184) (end 19.134 76.538) (width 1) (layer F.Cu) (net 9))
 (segment (start 19.134 83.124) (end 20.132 83.124) (width 1) (layer F.Cu) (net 9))
 (segment (start 20.828 83.82) (end 20.828 86.755) (width 1) (layer F.Cu) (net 9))
 (segment (start 20.132 83.124) (end 20.828 83.82) (width 1) (layer F.Cu) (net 9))
 (segment (start 20.828 86.755) (end 22.606 86.755) (width 1) (layer F.Cu) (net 9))
 (segment (start 24.13 86.755) (end 24.271 86.614) (width 1) (layer F.Cu) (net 9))
 (segment (start 22.606 86.755) (end 24.13 86.755) (width 1) (layer F.Cu) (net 9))
 (segment (start 25.92 74.88) (end 26.035 74.995) (width 0.2) (layer F.Cu) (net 4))
 (segment (start 25.92 72.644) (end 25.92 74.88) (width 0.2) (layer F.Cu) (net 4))
 (segment (start 26.035 74.995) (end 26.035 76.835) (width 0.2) (layer F.Cu) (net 4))
 (segment (start 25.36501 77.50499) (end 25.36501 82.18999) (width 0.2) (layer F.Cu) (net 4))
 (segment (start 25.36501 82.18999) (end 25.259 82.296) (width 0.2) (layer F.Cu) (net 4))
 (segment (start 26.035 76.835) (end 25.36501 77.50499) (width 0.2) (layer F.Cu) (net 4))
 (segment (start 25.259 82.296) (end 26.936 82.296) (width 0.2) (layer F.Cu) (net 4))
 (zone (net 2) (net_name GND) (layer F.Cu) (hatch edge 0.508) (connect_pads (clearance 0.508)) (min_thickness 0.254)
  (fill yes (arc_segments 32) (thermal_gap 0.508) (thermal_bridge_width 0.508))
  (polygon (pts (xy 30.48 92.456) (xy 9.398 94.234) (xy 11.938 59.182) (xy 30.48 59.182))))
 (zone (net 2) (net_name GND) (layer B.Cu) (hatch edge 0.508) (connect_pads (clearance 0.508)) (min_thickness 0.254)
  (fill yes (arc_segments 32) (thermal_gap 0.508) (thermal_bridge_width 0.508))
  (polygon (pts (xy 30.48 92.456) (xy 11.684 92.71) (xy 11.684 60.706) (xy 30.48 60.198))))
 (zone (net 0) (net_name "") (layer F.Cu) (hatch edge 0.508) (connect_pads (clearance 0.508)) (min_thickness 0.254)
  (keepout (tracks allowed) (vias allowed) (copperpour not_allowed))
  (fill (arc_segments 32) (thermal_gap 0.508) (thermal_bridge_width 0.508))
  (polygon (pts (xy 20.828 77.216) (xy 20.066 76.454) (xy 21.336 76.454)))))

